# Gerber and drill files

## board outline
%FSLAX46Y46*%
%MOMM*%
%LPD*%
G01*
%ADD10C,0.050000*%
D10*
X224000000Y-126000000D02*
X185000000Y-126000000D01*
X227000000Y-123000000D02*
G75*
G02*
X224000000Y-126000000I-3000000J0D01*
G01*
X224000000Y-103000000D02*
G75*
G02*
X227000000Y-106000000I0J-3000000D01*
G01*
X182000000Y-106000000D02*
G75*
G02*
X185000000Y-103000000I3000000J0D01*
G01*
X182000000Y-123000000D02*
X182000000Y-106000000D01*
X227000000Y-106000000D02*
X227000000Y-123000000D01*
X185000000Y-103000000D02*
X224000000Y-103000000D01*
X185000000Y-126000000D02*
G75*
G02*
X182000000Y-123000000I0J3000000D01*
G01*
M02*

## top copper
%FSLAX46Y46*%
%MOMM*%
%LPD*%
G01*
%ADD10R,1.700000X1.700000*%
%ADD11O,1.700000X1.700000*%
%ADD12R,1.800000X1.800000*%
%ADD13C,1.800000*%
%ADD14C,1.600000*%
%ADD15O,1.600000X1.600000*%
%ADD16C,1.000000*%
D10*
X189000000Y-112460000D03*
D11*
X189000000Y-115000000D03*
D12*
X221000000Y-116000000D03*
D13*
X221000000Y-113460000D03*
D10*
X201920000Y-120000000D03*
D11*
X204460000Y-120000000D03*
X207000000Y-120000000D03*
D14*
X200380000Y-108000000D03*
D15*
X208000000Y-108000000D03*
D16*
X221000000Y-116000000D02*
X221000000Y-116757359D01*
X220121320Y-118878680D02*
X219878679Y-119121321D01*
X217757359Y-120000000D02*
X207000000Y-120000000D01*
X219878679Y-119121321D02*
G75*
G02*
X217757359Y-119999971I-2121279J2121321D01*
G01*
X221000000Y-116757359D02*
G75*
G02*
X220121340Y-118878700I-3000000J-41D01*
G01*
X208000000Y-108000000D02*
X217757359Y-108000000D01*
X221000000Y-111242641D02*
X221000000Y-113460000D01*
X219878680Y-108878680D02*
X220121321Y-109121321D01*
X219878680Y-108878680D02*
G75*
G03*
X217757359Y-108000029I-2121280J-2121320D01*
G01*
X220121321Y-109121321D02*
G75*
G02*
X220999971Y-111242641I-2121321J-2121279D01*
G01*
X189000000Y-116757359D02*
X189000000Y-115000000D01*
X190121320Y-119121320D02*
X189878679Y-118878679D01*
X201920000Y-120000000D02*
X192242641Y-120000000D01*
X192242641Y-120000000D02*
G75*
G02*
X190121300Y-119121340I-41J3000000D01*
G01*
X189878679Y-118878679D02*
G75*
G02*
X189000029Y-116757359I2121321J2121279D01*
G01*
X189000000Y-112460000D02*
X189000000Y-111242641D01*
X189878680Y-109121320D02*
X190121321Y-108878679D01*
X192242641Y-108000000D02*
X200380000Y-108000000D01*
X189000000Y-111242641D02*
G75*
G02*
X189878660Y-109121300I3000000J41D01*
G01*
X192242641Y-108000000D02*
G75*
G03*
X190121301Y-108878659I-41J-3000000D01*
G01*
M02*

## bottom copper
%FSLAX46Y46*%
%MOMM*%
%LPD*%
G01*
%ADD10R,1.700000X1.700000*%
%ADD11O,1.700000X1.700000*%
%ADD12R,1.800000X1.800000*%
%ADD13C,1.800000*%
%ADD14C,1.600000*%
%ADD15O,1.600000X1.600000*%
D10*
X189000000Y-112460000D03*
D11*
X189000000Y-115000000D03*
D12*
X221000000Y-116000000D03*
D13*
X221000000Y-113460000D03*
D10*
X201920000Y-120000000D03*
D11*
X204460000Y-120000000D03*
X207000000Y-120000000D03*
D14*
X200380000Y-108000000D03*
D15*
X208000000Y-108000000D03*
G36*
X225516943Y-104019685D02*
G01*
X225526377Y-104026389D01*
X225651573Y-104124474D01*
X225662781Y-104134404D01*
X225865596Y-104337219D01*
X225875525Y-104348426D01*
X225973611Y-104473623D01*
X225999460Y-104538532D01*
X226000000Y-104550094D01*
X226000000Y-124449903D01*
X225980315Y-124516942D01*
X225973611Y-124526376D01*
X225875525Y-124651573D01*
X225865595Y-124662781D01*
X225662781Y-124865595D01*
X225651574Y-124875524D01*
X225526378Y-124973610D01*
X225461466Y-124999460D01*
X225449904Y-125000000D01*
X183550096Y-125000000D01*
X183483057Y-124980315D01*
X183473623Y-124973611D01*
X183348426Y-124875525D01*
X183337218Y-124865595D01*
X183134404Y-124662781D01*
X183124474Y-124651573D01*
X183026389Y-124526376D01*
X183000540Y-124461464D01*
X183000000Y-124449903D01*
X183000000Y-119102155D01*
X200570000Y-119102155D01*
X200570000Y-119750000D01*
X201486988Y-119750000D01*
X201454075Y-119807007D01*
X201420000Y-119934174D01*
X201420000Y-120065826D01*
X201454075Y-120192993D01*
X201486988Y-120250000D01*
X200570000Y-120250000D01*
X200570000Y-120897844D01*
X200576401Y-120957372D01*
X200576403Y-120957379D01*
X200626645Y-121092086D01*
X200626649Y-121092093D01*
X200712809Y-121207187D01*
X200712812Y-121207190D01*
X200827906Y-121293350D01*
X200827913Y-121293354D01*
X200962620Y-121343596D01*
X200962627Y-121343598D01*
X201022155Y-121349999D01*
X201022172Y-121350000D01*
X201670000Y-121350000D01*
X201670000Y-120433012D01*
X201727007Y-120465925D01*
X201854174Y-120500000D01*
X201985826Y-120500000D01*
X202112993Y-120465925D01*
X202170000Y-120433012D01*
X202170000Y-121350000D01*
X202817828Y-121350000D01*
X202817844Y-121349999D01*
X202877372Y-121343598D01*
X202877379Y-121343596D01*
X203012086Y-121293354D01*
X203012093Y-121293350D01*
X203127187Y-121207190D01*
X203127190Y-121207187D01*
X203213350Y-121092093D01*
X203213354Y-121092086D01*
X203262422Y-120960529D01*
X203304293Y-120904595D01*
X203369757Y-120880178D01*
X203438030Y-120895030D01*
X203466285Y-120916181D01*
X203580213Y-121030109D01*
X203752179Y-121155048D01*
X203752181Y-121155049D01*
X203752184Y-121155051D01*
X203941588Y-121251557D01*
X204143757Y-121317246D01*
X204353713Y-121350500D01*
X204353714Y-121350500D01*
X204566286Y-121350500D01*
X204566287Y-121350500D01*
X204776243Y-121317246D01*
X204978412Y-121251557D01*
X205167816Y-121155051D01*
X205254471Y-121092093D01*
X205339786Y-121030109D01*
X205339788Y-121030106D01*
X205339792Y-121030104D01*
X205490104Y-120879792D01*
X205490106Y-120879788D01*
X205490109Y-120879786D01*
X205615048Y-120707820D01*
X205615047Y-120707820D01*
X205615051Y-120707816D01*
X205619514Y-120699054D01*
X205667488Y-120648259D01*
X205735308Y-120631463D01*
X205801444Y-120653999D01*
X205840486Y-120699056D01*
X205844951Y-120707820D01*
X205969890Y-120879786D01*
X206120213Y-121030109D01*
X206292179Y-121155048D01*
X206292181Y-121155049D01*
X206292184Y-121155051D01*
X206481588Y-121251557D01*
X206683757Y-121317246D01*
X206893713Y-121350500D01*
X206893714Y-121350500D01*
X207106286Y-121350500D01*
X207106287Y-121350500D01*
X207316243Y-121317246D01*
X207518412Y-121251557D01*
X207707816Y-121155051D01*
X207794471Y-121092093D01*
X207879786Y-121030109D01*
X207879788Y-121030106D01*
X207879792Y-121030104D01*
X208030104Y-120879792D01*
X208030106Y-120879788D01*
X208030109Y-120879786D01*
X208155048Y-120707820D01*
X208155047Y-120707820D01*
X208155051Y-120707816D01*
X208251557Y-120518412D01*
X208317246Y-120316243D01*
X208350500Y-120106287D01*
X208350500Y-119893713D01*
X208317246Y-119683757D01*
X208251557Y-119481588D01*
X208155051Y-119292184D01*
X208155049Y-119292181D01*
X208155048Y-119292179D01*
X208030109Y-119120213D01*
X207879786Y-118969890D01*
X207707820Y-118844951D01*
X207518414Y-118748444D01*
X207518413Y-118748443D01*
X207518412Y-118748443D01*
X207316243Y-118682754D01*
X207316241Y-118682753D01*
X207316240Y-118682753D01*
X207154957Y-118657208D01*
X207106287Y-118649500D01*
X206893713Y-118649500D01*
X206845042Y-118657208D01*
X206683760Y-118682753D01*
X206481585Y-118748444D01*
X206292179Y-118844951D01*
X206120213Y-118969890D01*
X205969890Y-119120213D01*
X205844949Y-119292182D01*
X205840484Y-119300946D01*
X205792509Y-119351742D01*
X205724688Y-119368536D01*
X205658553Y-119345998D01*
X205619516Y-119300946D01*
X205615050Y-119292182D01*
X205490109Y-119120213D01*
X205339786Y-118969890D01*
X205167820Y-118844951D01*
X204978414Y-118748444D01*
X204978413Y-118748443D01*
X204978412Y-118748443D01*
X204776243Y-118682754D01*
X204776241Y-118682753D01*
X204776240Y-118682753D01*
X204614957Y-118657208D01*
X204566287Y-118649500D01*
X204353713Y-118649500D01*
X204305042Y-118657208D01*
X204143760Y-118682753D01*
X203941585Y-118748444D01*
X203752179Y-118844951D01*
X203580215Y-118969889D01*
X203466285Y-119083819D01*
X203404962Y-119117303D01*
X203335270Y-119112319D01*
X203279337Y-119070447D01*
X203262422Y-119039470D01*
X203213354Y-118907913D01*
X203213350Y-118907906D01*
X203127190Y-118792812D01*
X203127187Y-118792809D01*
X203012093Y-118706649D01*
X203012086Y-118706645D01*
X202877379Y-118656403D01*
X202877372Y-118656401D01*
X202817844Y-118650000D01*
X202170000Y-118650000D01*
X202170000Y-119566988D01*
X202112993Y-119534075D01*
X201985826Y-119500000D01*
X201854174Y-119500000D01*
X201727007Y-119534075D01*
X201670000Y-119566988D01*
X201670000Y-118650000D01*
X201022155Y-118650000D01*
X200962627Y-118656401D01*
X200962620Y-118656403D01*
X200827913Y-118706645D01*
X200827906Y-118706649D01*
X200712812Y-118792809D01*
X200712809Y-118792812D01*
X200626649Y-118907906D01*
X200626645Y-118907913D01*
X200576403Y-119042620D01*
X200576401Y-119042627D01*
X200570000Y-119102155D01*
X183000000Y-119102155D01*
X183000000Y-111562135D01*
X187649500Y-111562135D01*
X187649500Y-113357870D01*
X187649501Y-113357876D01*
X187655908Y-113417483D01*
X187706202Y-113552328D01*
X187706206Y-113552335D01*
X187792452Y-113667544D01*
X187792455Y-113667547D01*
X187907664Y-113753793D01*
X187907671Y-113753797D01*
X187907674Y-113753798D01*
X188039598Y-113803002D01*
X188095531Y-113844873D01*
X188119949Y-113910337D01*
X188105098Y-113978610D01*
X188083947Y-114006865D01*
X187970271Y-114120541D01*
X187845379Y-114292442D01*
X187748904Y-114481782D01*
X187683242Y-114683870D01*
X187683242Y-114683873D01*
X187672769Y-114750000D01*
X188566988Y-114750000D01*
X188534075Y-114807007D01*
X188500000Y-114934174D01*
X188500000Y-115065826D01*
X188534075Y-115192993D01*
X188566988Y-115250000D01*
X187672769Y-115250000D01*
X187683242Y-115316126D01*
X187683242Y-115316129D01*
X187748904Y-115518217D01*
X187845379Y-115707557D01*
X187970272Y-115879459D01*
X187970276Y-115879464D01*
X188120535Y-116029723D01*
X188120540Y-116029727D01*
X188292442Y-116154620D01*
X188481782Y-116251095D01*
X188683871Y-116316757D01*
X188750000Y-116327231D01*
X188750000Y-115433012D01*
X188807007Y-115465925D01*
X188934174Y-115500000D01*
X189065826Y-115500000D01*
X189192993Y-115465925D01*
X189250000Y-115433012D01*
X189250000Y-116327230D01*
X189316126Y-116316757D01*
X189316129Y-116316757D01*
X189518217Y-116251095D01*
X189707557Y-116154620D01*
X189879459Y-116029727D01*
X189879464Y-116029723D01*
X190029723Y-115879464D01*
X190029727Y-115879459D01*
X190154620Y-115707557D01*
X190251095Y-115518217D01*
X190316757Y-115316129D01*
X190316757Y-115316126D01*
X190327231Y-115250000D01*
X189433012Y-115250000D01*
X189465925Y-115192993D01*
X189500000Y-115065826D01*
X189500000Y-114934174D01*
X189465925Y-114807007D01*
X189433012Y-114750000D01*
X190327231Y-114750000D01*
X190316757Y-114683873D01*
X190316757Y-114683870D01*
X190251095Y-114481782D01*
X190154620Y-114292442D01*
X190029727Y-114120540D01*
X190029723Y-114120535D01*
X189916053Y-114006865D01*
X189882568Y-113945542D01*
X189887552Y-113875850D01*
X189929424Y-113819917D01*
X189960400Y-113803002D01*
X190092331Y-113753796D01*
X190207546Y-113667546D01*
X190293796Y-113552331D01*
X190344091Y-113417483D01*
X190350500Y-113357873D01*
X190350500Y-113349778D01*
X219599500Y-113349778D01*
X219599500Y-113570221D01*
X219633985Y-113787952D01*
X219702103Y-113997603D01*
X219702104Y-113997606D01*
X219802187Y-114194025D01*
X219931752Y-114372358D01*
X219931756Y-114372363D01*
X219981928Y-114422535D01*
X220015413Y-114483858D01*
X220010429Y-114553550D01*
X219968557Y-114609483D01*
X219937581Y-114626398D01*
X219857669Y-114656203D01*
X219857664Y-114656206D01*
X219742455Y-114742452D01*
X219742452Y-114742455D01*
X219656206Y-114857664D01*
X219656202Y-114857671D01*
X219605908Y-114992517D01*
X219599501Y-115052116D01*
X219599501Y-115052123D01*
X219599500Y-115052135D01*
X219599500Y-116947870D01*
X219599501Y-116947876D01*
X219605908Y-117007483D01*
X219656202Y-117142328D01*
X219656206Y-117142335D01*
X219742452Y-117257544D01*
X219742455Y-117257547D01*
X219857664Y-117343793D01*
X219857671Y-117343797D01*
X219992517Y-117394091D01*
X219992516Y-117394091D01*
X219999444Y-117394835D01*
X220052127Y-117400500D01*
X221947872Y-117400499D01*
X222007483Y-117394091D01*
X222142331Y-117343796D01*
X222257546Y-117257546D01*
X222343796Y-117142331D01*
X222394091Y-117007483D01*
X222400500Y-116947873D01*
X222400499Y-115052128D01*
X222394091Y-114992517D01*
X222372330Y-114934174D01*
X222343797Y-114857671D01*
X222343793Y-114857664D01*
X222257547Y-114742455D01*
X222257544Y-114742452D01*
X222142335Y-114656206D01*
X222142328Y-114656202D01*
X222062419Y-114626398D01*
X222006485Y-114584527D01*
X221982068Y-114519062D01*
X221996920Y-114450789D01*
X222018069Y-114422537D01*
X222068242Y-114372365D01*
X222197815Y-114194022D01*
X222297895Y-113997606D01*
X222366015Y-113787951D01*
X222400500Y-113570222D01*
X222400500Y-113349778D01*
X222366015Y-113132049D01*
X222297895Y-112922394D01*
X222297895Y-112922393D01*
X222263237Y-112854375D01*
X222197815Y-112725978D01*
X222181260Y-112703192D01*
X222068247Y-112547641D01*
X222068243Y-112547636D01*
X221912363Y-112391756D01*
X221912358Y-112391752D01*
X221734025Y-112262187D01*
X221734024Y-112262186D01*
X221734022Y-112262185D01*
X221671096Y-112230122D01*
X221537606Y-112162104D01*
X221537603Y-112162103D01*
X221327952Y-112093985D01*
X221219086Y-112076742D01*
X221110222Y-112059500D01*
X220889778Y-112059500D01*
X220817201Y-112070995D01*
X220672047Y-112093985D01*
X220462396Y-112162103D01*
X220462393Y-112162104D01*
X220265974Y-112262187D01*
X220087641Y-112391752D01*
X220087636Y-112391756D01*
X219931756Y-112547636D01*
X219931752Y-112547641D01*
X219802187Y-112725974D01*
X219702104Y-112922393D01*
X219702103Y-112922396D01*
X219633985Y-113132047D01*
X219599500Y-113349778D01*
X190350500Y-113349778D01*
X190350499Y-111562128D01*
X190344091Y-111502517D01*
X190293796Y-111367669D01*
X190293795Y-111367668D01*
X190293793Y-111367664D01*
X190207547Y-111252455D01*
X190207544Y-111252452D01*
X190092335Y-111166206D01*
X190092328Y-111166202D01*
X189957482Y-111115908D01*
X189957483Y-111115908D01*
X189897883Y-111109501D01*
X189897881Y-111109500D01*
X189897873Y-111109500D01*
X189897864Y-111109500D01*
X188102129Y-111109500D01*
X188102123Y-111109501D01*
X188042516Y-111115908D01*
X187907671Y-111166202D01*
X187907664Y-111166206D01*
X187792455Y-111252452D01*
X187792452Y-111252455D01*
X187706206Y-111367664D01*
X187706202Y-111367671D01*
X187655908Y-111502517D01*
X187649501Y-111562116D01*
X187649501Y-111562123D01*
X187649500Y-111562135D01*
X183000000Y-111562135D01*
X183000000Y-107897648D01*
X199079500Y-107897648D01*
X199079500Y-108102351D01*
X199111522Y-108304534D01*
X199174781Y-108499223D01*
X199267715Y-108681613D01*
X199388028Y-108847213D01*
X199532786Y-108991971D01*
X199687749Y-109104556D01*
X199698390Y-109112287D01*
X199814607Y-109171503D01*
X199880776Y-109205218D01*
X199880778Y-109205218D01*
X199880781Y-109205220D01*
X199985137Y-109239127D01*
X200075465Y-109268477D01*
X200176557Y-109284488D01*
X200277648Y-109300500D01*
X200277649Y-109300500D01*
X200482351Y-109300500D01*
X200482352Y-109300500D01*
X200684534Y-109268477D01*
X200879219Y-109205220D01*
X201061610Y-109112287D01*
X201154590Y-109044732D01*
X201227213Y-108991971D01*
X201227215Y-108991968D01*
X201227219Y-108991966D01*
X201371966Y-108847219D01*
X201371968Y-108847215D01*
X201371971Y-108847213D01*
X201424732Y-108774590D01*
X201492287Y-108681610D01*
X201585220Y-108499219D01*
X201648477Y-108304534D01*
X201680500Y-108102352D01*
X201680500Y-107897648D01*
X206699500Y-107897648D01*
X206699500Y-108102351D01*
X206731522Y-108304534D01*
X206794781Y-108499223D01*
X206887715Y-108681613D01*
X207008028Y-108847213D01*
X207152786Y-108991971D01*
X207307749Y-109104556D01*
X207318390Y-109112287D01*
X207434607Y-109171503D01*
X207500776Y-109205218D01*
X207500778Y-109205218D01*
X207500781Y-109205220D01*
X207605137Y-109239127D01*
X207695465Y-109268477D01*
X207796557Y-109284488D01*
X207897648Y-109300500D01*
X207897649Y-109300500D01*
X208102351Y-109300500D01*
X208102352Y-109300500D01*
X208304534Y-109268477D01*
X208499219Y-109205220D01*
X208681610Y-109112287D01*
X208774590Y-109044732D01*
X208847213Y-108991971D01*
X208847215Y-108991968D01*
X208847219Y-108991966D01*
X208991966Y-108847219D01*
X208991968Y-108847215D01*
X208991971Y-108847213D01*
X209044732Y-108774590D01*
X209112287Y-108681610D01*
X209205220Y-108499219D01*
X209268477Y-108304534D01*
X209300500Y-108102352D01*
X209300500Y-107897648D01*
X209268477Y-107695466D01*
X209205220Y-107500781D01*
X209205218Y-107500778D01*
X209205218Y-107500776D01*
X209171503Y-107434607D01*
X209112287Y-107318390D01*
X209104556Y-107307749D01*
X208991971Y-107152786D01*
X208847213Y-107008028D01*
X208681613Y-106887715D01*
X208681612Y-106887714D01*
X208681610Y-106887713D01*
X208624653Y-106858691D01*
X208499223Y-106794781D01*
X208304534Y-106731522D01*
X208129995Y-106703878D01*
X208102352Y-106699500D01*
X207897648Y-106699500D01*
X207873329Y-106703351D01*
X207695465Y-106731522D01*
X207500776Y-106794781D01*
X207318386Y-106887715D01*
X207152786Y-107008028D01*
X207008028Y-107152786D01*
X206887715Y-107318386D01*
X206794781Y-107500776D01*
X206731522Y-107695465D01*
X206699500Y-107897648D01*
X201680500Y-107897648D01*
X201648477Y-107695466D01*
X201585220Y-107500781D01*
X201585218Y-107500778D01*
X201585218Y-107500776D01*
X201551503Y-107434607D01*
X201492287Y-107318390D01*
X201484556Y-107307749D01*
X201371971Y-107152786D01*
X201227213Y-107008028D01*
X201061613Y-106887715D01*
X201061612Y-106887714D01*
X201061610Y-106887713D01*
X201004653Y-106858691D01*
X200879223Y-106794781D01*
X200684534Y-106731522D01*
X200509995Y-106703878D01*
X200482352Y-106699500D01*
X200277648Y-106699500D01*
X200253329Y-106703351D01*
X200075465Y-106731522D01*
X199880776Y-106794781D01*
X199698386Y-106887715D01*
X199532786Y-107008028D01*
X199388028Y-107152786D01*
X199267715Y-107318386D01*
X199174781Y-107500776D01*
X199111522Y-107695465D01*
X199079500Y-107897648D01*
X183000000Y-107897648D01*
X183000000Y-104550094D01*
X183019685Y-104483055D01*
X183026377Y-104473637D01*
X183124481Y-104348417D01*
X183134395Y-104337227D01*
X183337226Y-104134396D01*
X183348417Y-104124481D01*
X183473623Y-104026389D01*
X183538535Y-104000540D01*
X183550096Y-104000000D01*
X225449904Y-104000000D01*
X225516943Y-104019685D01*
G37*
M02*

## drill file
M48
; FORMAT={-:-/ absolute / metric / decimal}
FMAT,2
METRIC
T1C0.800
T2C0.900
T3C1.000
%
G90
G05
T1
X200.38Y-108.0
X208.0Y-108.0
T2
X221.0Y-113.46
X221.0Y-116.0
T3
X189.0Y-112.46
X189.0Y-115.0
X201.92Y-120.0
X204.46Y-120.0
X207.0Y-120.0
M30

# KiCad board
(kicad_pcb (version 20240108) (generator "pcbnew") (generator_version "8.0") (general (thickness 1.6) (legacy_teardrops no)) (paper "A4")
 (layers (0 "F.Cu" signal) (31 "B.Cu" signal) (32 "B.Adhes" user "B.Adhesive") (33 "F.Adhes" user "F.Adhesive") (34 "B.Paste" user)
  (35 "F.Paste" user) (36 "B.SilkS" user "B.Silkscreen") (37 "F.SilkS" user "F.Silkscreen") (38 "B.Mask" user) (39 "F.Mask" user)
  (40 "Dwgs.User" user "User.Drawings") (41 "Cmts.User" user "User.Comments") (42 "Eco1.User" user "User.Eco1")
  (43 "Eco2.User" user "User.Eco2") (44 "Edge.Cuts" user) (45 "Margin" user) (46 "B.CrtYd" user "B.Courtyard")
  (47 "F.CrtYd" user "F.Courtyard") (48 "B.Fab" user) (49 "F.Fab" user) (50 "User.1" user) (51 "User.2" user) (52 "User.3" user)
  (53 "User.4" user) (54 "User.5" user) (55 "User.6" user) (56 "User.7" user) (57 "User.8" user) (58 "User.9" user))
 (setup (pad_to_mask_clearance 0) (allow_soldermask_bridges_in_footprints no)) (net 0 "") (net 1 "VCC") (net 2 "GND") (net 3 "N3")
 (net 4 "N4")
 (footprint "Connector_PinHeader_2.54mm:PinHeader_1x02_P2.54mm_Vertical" (layer "F.Cu") (at 189 112.46)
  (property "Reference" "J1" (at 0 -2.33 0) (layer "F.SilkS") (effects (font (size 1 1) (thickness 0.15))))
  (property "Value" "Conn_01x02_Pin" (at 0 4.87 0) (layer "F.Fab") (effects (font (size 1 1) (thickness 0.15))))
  (pad "1" thru_hole rect (at 0 0) (size 1.7 1.7) (drill 1) (layers "*.Cu" "*.Mask") (remove_unused_layers no) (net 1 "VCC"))
  (pad "2" thru_hole oval (at 0 2.54) (size 1.7 1.7) (drill 1) (layers "*.Cu" "*.Mask") (remove_unused_layers no) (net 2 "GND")))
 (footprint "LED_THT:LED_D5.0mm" (layer "F.Cu") (at 221 116 90)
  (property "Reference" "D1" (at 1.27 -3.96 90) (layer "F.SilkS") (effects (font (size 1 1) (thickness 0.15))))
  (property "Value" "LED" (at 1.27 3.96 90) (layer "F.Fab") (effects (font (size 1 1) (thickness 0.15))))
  (pad "1" thru_hole rect (at 0 0 90) (size 1.8 1.8) (drill 0.9) (layers "*.Cu" "*.Mask") (remove_unused_layers no) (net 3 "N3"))
  (pad "2" thru_hole circle (at 2.54 0 90) (size 1.8 1.8) (drill 0.9) (layers "*.Cu" "*.Mask") (remove_unused_layers no) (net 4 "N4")))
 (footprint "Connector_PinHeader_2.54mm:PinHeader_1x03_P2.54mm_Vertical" (layer "F.Cu") (at 201.92 120 90)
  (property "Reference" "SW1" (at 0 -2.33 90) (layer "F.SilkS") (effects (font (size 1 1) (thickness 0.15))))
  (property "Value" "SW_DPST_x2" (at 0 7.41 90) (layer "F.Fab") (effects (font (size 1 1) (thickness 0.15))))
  (pad "1" thru_hole rect (at 0 0 90) (size 1.7 1.7) (drill 1) (layers "*.Cu" "*.Mask") (remove_unused_layers no) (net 2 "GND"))
  (pad "2" thru_hole oval (at 0 2.54 90) (size 1.7 1.7) (drill 1) (layers "*.Cu" "*.Mask") (remove_unused_layers no))
  (pad "3" thru_hole oval (at 0 5.08 90) (size 1.7 1.7) (drill 1) (layers "*.Cu" "*.Mask") (remove_unused_layers no) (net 3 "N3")))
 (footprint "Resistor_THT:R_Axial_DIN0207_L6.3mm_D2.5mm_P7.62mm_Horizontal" (layer "F.Cu") (at 200.38 108)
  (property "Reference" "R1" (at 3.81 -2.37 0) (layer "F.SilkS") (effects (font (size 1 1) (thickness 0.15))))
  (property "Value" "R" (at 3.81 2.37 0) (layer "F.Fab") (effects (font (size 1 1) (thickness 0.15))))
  (pad "1" thru_hole circle (at 0 0) (size 1.6 1.6) (drill 0.8) (layers "*.Cu" "*.Mask") (remove_unused_layers no) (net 1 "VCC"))
  (pad "2" thru_hole oval (at 7.62 0) (size 1.6 1.6) (drill 0.8) (layers "*.Cu" "*.Mask") (remove_unused_layers no) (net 4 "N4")))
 (gr_line (start 224 126) (end 185 126) (stroke (width 0.05) (type default)) (layer "Edge.Cuts"))
 (gr_arc (start 227 123) (mid 226.12132 125.12132) (end 224 126) (stroke (width 0.05) (type default)) (layer "Edge.Cuts"))
 (gr_arc (start 224 103) (mid 226.12132 103.87868) (end 227 106) (stroke (width 0.05) (type default)) (layer "Edge.Cuts"))
 (gr_arc (start 182 106) (mid 182.87868 103.87868) (end 185 103) (stroke (width 0.05) (type default)) (layer "Edge.Cuts"))
 (gr_line (start 182 123) (end 182 106) (stroke (width 0.05) (type default)) (layer "Edge.Cuts"))
 (gr_line (start 227 106) (end 227 123) (stroke (width 0.05) (type default)) (layer "Edge.Cuts"))
 (gr_line (start 185 103) (end 224 103) (stroke (width 0.05) (type default)) (layer "Edge.Cuts"))
 (gr_arc (start 185 126) (mid 182.87868 125.12132) (end 182 123) (stroke (width 0.05) (type default)) (layer "Edge.Cuts"))
 (segment (start 221 116) (end 221 116.757359) (width 1) (layer "F.Cu") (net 3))
 (segment (start 220.12132 118.87868) (end 219.878679 119.121321) (width 1) (layer "F.Cu") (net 3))
 (segment (start 217.757359 120) (end 207 120) (width 1) (layer "F.Cu") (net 3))
 (arc (start 219.878679 119.121321) (mid 218.905409 119.771639) (end 217.757359 120) (width 1) (layer "F.Cu") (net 3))
 (arc (start 221 116.757359) (mid 220.771638 117.90541) (end 220.12132 118.87868) (width 1) (layer "F.Cu") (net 3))
 (segment (start 208 108) (end 217.757359 108) (width 1) (layer "F.Cu") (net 4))
 (segment (start 221 111.242641) (end 221 113.46) (width 1) (layer "F.Cu") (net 4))
 (segment (start 219.87868 108.87868) (end 220.121321 109.121321) (width 1) (layer "F.Cu") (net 4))
 (arc (start 219.87868 108.87868) (mid 218.90541 108.228361) (end 217.757359 108) (width 1) (layer "F.Cu") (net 4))
 (arc (start 220.121321 109.121321) (mid 220.771639 110.094591) (end 221 111.242641) (width 1) (layer "F.Cu") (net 4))
 (segment (start 189 116.757359) (end 189 115) (width 1) (layer "F.Cu") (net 2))
 (segment (start 190.12132 119.12132) (end 189.878679 118.878679) (width 1) (layer "F.Cu") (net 2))
 (segment (start 201.92 120) (end 192.242641 120) (width 1) (layer "F.Cu") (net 2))
 (arc (start 192.242641 120) (mid 191.09459 119.771638) (end 190.12132 119.12132) (width 1) (layer "F.Cu") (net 2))
 (arc (start 189.878679 118.878679) (mid 189.228361 117.905409) (end 189 116.757359) (width 1) (layer "F.Cu") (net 2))
 (segment (start 189 112.46) (end 189 111.242641) (width 1) (layer "F.Cu") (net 1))
 (segment (start 189.87868 109.12132) (end 190.121321 108.878679) (width 1) (layer "F.Cu") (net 1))
 (segment (start 192.242641 108) (end 200.38 108) (width 1) (layer "F.Cu") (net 1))
 (arc (start 189 111.242641) (mid 189.228362 110.09459) (end 189.87868 109.12132) (width 1) (layer "F.Cu") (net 1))
 (arc (start 192.242641 108) (mid 191.094591 108.228361) (end 190.121321 108.878679) (width 1) (layer "F.Cu") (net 1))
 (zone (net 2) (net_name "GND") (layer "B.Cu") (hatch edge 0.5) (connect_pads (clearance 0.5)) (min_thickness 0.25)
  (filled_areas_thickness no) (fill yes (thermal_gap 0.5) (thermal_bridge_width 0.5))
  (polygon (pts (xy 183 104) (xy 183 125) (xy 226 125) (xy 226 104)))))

